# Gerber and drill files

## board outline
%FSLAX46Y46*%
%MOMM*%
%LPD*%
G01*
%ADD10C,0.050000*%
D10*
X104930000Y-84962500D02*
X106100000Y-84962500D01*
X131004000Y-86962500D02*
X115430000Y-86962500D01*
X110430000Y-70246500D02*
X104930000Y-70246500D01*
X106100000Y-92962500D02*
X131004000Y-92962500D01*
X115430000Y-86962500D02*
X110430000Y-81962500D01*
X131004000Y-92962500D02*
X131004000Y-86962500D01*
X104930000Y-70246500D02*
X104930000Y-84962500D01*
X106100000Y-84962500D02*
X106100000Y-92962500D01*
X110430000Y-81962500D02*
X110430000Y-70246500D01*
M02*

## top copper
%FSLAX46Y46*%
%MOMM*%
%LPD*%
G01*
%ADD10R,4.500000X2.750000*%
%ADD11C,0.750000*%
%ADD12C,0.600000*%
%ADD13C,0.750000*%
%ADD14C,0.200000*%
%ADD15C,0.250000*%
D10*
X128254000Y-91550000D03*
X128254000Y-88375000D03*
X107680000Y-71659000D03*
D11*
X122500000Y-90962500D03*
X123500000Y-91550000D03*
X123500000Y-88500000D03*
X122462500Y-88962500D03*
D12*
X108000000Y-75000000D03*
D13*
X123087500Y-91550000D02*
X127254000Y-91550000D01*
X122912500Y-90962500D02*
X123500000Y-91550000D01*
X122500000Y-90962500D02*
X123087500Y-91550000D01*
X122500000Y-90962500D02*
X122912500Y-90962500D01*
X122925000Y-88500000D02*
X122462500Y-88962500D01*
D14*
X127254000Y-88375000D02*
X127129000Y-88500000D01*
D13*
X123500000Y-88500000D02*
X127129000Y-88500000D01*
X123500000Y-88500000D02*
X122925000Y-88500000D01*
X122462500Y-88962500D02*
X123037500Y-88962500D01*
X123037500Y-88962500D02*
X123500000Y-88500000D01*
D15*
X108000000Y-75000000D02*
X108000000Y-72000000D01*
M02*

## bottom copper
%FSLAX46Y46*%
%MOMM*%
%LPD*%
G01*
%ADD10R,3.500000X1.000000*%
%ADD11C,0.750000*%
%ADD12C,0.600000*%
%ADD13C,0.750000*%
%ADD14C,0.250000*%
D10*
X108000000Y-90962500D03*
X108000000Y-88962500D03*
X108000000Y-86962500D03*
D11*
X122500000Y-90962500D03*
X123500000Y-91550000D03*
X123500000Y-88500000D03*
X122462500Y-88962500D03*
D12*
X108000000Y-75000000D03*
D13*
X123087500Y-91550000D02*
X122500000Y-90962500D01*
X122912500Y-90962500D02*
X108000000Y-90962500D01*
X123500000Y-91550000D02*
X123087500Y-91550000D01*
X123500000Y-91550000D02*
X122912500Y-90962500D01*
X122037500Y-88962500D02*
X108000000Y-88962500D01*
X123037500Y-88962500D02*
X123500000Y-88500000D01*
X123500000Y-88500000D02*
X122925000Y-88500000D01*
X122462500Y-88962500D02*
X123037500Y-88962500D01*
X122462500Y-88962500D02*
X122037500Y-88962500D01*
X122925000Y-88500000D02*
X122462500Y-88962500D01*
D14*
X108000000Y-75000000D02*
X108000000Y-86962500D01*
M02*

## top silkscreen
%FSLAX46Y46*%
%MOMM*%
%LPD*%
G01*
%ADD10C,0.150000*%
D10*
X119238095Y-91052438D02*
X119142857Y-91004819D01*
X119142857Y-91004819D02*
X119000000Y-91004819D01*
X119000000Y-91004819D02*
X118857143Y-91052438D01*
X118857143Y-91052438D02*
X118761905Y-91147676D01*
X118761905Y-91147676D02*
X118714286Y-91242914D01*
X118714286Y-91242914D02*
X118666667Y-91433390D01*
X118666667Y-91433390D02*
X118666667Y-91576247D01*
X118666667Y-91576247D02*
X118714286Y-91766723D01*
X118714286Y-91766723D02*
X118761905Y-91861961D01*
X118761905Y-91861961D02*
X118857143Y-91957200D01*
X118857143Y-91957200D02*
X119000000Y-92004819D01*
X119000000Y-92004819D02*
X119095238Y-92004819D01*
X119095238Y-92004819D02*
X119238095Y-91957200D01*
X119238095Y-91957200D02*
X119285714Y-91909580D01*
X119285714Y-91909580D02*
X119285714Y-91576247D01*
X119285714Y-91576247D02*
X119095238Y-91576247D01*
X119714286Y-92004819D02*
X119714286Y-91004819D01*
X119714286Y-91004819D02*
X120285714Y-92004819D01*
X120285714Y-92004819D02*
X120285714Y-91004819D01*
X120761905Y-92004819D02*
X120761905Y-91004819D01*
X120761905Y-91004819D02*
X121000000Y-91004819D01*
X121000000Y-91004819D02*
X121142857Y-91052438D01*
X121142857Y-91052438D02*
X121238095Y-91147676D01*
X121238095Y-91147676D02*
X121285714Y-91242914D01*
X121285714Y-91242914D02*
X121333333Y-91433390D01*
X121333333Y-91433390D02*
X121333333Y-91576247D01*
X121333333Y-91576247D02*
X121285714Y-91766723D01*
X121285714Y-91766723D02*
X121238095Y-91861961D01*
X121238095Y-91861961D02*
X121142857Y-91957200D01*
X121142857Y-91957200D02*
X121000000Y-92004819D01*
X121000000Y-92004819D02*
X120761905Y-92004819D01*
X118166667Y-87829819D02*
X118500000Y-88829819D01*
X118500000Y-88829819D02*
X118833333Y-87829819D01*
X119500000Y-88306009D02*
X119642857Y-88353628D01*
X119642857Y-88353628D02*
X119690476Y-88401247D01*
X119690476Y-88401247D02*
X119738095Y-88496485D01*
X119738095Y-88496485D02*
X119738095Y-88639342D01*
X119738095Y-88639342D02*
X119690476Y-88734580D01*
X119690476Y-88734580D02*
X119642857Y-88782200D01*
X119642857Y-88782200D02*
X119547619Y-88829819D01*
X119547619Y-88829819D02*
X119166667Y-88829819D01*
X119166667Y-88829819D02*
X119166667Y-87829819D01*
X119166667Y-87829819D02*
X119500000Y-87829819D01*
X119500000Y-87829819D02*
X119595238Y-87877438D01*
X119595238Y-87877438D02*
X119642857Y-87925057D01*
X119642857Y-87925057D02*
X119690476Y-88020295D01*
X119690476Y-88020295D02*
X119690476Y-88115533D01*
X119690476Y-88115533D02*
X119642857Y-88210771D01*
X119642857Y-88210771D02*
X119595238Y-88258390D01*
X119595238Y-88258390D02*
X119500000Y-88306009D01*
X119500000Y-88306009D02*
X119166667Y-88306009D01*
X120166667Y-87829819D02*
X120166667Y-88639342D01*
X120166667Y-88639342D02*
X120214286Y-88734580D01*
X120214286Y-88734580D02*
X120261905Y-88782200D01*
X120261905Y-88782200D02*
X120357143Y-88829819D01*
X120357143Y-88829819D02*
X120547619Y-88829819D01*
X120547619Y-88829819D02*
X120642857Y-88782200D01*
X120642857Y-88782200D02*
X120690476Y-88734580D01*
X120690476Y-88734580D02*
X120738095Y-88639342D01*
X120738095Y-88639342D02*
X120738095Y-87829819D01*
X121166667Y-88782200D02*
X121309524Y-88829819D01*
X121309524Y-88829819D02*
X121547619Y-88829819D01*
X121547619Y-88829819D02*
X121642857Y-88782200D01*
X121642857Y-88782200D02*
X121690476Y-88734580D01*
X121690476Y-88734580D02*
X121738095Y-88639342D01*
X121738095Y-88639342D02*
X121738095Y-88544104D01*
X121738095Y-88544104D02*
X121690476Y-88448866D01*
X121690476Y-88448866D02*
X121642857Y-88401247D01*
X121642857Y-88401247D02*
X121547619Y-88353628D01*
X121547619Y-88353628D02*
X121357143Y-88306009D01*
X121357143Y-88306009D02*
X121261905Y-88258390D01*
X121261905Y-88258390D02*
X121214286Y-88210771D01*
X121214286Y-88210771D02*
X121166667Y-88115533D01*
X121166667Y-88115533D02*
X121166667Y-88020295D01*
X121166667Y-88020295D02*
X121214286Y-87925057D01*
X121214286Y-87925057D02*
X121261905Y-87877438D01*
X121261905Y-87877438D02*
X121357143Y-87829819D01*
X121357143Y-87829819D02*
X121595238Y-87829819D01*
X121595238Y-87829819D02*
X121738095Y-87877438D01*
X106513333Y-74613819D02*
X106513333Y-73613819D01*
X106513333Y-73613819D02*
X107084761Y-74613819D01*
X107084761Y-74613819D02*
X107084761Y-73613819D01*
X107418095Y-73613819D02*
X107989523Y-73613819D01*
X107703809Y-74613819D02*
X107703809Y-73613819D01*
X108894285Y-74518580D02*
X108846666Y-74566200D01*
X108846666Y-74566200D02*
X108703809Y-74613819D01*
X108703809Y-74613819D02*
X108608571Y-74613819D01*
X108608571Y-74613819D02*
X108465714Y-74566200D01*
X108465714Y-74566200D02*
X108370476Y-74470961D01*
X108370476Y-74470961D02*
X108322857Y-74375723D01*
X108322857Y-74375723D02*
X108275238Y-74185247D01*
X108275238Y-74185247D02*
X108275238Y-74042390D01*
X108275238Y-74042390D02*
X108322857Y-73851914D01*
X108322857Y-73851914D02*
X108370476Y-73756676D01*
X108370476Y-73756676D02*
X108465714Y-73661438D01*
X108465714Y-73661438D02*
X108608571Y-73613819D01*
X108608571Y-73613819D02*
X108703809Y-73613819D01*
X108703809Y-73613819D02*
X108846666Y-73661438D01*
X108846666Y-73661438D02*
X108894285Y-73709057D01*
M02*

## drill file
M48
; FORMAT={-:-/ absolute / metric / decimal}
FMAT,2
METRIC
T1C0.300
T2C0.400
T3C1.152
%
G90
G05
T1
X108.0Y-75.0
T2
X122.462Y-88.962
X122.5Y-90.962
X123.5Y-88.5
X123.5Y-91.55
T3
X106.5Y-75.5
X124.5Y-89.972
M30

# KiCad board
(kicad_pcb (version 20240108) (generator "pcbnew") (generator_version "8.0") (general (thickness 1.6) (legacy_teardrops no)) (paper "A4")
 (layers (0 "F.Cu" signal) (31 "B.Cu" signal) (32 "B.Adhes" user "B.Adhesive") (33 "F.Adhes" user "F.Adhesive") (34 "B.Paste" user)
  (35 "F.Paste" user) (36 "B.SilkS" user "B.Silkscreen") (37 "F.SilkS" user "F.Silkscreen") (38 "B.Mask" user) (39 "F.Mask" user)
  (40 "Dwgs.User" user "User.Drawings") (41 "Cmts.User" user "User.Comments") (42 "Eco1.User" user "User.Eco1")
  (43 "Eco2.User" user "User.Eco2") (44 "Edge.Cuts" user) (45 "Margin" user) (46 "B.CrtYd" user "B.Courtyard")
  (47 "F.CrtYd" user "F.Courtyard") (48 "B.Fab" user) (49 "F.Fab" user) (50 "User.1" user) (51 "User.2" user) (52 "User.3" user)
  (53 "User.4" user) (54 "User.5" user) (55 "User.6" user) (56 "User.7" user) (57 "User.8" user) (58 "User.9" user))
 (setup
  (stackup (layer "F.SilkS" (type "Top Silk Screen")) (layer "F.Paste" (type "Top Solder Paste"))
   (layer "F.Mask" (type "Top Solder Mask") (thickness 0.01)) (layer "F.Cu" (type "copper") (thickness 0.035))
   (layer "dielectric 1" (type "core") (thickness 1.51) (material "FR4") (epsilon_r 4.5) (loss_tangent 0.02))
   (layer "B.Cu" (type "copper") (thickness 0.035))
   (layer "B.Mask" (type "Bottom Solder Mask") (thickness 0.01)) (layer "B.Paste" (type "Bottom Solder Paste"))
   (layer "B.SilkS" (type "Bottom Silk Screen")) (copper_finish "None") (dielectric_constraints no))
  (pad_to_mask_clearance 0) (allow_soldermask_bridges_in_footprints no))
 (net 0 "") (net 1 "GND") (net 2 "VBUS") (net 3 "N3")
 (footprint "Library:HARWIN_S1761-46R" (layer "F.Cu") (at 128.254 91.55 90)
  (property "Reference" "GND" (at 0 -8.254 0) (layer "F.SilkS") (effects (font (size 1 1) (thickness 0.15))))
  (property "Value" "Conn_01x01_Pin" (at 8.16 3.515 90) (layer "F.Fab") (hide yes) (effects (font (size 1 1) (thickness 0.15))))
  (pad "1" smd rect (at 0 0 90) (size 2.75 4.5) (layers "F.Cu" "F.Paste" "F.Mask") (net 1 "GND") (solder_mask_margin 0.102)))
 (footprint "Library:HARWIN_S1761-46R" (layer "F.Cu") (at 128.254 88.375 90)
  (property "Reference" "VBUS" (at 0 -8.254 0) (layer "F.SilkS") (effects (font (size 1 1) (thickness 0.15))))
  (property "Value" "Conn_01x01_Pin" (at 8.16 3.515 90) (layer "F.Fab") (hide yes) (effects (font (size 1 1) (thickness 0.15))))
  (pad "1" smd rect (at 0 0 90) (size 2.75 4.5) (layers "F.Cu" "F.Paste" "F.Mask") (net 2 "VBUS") (solder_mask_margin 0.102)))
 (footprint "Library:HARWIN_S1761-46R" (layer "F.Cu") (at 107.68 71.659 -90)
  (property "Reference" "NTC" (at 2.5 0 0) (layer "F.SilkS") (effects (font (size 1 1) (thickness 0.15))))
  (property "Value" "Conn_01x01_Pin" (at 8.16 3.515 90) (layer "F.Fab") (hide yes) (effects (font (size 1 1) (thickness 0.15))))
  (pad "1" smd rect (at 0 0 270) (size 2.75 4.5) (layers "F.Cu" "F.Paste" "F.Mask") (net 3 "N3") (solder_mask_margin 0.102)))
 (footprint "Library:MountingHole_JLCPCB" (layer "F.Cu") (at 106.5 75.5)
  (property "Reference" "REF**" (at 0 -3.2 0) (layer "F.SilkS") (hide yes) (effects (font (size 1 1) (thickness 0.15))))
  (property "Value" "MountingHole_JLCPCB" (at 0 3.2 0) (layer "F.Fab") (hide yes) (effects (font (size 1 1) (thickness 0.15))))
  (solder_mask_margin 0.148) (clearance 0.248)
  (pad "" np_thru_hole circle (at 0 0) (size 1.152 1.152) (drill 1.152) (layers "F&B.Cu" "*.Mask")))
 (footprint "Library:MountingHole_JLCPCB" (layer "F.Cu") (at 124.5 90)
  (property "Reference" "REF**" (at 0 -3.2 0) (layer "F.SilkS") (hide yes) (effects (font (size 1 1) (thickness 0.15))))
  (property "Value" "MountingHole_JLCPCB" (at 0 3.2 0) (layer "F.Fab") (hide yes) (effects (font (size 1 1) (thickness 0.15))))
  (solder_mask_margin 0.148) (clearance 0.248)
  (pad "" np_thru_hole circle (at 0 -0.0275) (size 1.152 1.152) (drill 1.152) (layers "F&B.Cu" "*.Mask")))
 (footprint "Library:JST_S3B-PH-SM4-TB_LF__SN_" (layer "B.Cu") (at 108 88.9625 -90)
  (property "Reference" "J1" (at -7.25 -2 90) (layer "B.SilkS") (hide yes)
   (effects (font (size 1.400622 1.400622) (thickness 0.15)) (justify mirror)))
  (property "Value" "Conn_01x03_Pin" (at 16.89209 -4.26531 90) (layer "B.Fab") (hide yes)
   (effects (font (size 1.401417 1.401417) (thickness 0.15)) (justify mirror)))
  (pad "1" smd rect (at 2 0 270) (size 1 3.5) (layers "B.Cu" "B.Paste" "B.Mask") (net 1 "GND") (solder_mask_margin 0.102))
  (pad "2" smd rect (at 0 0 270) (size 1 3.5) (layers "B.Cu" "B.Paste" "B.Mask") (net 2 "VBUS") (solder_mask_margin 0.102))
  (pad "3" smd rect (at -2 0 270) (size 1 3.5) (layers "B.Cu" "B.Paste" "B.Mask") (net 3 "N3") (solder_mask_margin 0.102)))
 (gr_line (start 104.93 84.9625) (end 106.1 84.9625) (stroke (width 0.05) (type default)) (layer "Edge.Cuts"))
 (gr_line (start 131.004 86.9625) (end 115.43 86.9625) (stroke (width 0.05) (type default)) (layer "Edge.Cuts"))
 (gr_line (start 110.43 70.2465) (end 104.93 70.2465) (stroke (width 0.05) (type default)) (layer "Edge.Cuts"))
 (gr_line (start 106.1 92.9625) (end 131.004 92.9625) (stroke (width 0.05) (type default)) (layer "Edge.Cuts"))
 (gr_line (start 115.43 86.9625) (end 110.43 81.9625) (stroke (width 0.05) (type default)) (layer "Edge.Cuts"))
 (gr_line (start 131.004 92.9625) (end 131.004 86.9625) (stroke (width 0.05) (type default)) (layer "Edge.Cuts"))
 (gr_line (start 104.93 70.2465) (end 104.93 84.9625) (stroke (width 0.05) (type default)) (layer "Edge.Cuts"))
 (gr_line (start 106.1 84.9625) (end 106.1 92.9625) (stroke (width 0.05) (type default)) (layer "Edge.Cuts"))
 (gr_line (start 110.43 81.9625) (end 110.43 70.2465) (stroke (width 0.05) (type default)) (layer "Edge.Cuts"))
 (segment (start 123.0875 91.55) (end 127.254 91.55) (width 0.75) (layer "F.Cu") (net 1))
 (segment (start 122.9125 90.9625) (end 123.5 91.55) (width 0.75) (layer "F.Cu") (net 1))
 (segment (start 122.5 90.9625) (end 123.0875 91.55) (width 0.75) (layer "F.Cu") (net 1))
 (segment (start 122.5 90.9625) (end 122.9125 90.9625) (width 0.75) (layer "F.Cu") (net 1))
 (via (at 122.5 90.9625) (size 0.75) (drill 0.4) (layers "F.Cu" "B.Cu") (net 1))
 (via (at 123.5 91.55) (size 0.75) (drill 0.4) (layers "F.Cu" "B.Cu") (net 1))
 (segment (start 123.0875 91.55) (end 122.5 90.9625) (width 0.75) (layer "B.Cu") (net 1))
 (segment (start 122.9125 90.9625) (end 108 90.9625) (width 0.75) (layer "B.Cu") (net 1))
 (segment (start 123.5 91.55) (end 123.0875 91.55) (width 0.75) (layer "B.Cu") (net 1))
 (segment (start 123.5 91.55) (end 122.9125 90.9625) (width 0.75) (layer "B.Cu") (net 1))
 (segment (start 122.925 88.5) (end 122.4625 88.9625) (width 0.75) (layer "F.Cu") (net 2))
 (segment (start 127.254 88.375) (end 127.129 88.5) (width 0.2) (layer "F.Cu") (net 2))
 (segment (start 123.5 88.5) (end 127.129 88.5) (width 0.75) (layer "F.Cu") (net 2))
 (segment (start 123.5 88.5) (end 122.925 88.5) (width 0.75) (layer "F.Cu") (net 2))
 (segment (start 122.4625 88.9625) (end 123.0375 88.9625) (width 0.75) (layer "F.Cu") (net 2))
 (segment (start 123.0375 88.9625) (end 123.5 88.5) (width 0.75) (layer "F.Cu") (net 2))
 (via (at 123.5 88.5) (size 0.75) (drill 0.4) (layers "F.Cu" "B.Cu") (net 2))
 (via (at 122.4625 88.9625) (size 0.75) (drill 0.4) (layers "F.Cu" "B.Cu") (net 2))
 (segment (start 122.0375 88.9625) (end 108 88.9625) (width 0.75) (layer "B.Cu") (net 2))
 (segment (start 123.0375 88.9625) (end 123.5 88.5) (width 0.75) (layer "B.Cu") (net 2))
 (segment (start 123.5 88.5) (end 122.925 88.5) (width 0.75) (layer "B.Cu") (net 2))
 (segment (start 122.4625 88.9625) (end 123.0375 88.9625) (width 0.75) (layer "B.Cu") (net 2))
 (segment (start 122.4625 88.9625) (end 122.0375 88.9625) (width 0.75) (layer "B.Cu") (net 2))
 (segment (start 122.925 88.5) (end 122.4625 88.9625) (width 0.75) (layer "B.Cu") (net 2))
 (segment (start 108 75) (end 108 72) (width 0.25) (layer "F.Cu") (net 3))
 (via (at 108 75) (size 0.6) (drill 0.3) (layers "F.Cu" "B.Cu") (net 3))
 (segment (start 108 75) (end 108 86.9625) (width 0.25) (layer "B.Cu") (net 3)))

